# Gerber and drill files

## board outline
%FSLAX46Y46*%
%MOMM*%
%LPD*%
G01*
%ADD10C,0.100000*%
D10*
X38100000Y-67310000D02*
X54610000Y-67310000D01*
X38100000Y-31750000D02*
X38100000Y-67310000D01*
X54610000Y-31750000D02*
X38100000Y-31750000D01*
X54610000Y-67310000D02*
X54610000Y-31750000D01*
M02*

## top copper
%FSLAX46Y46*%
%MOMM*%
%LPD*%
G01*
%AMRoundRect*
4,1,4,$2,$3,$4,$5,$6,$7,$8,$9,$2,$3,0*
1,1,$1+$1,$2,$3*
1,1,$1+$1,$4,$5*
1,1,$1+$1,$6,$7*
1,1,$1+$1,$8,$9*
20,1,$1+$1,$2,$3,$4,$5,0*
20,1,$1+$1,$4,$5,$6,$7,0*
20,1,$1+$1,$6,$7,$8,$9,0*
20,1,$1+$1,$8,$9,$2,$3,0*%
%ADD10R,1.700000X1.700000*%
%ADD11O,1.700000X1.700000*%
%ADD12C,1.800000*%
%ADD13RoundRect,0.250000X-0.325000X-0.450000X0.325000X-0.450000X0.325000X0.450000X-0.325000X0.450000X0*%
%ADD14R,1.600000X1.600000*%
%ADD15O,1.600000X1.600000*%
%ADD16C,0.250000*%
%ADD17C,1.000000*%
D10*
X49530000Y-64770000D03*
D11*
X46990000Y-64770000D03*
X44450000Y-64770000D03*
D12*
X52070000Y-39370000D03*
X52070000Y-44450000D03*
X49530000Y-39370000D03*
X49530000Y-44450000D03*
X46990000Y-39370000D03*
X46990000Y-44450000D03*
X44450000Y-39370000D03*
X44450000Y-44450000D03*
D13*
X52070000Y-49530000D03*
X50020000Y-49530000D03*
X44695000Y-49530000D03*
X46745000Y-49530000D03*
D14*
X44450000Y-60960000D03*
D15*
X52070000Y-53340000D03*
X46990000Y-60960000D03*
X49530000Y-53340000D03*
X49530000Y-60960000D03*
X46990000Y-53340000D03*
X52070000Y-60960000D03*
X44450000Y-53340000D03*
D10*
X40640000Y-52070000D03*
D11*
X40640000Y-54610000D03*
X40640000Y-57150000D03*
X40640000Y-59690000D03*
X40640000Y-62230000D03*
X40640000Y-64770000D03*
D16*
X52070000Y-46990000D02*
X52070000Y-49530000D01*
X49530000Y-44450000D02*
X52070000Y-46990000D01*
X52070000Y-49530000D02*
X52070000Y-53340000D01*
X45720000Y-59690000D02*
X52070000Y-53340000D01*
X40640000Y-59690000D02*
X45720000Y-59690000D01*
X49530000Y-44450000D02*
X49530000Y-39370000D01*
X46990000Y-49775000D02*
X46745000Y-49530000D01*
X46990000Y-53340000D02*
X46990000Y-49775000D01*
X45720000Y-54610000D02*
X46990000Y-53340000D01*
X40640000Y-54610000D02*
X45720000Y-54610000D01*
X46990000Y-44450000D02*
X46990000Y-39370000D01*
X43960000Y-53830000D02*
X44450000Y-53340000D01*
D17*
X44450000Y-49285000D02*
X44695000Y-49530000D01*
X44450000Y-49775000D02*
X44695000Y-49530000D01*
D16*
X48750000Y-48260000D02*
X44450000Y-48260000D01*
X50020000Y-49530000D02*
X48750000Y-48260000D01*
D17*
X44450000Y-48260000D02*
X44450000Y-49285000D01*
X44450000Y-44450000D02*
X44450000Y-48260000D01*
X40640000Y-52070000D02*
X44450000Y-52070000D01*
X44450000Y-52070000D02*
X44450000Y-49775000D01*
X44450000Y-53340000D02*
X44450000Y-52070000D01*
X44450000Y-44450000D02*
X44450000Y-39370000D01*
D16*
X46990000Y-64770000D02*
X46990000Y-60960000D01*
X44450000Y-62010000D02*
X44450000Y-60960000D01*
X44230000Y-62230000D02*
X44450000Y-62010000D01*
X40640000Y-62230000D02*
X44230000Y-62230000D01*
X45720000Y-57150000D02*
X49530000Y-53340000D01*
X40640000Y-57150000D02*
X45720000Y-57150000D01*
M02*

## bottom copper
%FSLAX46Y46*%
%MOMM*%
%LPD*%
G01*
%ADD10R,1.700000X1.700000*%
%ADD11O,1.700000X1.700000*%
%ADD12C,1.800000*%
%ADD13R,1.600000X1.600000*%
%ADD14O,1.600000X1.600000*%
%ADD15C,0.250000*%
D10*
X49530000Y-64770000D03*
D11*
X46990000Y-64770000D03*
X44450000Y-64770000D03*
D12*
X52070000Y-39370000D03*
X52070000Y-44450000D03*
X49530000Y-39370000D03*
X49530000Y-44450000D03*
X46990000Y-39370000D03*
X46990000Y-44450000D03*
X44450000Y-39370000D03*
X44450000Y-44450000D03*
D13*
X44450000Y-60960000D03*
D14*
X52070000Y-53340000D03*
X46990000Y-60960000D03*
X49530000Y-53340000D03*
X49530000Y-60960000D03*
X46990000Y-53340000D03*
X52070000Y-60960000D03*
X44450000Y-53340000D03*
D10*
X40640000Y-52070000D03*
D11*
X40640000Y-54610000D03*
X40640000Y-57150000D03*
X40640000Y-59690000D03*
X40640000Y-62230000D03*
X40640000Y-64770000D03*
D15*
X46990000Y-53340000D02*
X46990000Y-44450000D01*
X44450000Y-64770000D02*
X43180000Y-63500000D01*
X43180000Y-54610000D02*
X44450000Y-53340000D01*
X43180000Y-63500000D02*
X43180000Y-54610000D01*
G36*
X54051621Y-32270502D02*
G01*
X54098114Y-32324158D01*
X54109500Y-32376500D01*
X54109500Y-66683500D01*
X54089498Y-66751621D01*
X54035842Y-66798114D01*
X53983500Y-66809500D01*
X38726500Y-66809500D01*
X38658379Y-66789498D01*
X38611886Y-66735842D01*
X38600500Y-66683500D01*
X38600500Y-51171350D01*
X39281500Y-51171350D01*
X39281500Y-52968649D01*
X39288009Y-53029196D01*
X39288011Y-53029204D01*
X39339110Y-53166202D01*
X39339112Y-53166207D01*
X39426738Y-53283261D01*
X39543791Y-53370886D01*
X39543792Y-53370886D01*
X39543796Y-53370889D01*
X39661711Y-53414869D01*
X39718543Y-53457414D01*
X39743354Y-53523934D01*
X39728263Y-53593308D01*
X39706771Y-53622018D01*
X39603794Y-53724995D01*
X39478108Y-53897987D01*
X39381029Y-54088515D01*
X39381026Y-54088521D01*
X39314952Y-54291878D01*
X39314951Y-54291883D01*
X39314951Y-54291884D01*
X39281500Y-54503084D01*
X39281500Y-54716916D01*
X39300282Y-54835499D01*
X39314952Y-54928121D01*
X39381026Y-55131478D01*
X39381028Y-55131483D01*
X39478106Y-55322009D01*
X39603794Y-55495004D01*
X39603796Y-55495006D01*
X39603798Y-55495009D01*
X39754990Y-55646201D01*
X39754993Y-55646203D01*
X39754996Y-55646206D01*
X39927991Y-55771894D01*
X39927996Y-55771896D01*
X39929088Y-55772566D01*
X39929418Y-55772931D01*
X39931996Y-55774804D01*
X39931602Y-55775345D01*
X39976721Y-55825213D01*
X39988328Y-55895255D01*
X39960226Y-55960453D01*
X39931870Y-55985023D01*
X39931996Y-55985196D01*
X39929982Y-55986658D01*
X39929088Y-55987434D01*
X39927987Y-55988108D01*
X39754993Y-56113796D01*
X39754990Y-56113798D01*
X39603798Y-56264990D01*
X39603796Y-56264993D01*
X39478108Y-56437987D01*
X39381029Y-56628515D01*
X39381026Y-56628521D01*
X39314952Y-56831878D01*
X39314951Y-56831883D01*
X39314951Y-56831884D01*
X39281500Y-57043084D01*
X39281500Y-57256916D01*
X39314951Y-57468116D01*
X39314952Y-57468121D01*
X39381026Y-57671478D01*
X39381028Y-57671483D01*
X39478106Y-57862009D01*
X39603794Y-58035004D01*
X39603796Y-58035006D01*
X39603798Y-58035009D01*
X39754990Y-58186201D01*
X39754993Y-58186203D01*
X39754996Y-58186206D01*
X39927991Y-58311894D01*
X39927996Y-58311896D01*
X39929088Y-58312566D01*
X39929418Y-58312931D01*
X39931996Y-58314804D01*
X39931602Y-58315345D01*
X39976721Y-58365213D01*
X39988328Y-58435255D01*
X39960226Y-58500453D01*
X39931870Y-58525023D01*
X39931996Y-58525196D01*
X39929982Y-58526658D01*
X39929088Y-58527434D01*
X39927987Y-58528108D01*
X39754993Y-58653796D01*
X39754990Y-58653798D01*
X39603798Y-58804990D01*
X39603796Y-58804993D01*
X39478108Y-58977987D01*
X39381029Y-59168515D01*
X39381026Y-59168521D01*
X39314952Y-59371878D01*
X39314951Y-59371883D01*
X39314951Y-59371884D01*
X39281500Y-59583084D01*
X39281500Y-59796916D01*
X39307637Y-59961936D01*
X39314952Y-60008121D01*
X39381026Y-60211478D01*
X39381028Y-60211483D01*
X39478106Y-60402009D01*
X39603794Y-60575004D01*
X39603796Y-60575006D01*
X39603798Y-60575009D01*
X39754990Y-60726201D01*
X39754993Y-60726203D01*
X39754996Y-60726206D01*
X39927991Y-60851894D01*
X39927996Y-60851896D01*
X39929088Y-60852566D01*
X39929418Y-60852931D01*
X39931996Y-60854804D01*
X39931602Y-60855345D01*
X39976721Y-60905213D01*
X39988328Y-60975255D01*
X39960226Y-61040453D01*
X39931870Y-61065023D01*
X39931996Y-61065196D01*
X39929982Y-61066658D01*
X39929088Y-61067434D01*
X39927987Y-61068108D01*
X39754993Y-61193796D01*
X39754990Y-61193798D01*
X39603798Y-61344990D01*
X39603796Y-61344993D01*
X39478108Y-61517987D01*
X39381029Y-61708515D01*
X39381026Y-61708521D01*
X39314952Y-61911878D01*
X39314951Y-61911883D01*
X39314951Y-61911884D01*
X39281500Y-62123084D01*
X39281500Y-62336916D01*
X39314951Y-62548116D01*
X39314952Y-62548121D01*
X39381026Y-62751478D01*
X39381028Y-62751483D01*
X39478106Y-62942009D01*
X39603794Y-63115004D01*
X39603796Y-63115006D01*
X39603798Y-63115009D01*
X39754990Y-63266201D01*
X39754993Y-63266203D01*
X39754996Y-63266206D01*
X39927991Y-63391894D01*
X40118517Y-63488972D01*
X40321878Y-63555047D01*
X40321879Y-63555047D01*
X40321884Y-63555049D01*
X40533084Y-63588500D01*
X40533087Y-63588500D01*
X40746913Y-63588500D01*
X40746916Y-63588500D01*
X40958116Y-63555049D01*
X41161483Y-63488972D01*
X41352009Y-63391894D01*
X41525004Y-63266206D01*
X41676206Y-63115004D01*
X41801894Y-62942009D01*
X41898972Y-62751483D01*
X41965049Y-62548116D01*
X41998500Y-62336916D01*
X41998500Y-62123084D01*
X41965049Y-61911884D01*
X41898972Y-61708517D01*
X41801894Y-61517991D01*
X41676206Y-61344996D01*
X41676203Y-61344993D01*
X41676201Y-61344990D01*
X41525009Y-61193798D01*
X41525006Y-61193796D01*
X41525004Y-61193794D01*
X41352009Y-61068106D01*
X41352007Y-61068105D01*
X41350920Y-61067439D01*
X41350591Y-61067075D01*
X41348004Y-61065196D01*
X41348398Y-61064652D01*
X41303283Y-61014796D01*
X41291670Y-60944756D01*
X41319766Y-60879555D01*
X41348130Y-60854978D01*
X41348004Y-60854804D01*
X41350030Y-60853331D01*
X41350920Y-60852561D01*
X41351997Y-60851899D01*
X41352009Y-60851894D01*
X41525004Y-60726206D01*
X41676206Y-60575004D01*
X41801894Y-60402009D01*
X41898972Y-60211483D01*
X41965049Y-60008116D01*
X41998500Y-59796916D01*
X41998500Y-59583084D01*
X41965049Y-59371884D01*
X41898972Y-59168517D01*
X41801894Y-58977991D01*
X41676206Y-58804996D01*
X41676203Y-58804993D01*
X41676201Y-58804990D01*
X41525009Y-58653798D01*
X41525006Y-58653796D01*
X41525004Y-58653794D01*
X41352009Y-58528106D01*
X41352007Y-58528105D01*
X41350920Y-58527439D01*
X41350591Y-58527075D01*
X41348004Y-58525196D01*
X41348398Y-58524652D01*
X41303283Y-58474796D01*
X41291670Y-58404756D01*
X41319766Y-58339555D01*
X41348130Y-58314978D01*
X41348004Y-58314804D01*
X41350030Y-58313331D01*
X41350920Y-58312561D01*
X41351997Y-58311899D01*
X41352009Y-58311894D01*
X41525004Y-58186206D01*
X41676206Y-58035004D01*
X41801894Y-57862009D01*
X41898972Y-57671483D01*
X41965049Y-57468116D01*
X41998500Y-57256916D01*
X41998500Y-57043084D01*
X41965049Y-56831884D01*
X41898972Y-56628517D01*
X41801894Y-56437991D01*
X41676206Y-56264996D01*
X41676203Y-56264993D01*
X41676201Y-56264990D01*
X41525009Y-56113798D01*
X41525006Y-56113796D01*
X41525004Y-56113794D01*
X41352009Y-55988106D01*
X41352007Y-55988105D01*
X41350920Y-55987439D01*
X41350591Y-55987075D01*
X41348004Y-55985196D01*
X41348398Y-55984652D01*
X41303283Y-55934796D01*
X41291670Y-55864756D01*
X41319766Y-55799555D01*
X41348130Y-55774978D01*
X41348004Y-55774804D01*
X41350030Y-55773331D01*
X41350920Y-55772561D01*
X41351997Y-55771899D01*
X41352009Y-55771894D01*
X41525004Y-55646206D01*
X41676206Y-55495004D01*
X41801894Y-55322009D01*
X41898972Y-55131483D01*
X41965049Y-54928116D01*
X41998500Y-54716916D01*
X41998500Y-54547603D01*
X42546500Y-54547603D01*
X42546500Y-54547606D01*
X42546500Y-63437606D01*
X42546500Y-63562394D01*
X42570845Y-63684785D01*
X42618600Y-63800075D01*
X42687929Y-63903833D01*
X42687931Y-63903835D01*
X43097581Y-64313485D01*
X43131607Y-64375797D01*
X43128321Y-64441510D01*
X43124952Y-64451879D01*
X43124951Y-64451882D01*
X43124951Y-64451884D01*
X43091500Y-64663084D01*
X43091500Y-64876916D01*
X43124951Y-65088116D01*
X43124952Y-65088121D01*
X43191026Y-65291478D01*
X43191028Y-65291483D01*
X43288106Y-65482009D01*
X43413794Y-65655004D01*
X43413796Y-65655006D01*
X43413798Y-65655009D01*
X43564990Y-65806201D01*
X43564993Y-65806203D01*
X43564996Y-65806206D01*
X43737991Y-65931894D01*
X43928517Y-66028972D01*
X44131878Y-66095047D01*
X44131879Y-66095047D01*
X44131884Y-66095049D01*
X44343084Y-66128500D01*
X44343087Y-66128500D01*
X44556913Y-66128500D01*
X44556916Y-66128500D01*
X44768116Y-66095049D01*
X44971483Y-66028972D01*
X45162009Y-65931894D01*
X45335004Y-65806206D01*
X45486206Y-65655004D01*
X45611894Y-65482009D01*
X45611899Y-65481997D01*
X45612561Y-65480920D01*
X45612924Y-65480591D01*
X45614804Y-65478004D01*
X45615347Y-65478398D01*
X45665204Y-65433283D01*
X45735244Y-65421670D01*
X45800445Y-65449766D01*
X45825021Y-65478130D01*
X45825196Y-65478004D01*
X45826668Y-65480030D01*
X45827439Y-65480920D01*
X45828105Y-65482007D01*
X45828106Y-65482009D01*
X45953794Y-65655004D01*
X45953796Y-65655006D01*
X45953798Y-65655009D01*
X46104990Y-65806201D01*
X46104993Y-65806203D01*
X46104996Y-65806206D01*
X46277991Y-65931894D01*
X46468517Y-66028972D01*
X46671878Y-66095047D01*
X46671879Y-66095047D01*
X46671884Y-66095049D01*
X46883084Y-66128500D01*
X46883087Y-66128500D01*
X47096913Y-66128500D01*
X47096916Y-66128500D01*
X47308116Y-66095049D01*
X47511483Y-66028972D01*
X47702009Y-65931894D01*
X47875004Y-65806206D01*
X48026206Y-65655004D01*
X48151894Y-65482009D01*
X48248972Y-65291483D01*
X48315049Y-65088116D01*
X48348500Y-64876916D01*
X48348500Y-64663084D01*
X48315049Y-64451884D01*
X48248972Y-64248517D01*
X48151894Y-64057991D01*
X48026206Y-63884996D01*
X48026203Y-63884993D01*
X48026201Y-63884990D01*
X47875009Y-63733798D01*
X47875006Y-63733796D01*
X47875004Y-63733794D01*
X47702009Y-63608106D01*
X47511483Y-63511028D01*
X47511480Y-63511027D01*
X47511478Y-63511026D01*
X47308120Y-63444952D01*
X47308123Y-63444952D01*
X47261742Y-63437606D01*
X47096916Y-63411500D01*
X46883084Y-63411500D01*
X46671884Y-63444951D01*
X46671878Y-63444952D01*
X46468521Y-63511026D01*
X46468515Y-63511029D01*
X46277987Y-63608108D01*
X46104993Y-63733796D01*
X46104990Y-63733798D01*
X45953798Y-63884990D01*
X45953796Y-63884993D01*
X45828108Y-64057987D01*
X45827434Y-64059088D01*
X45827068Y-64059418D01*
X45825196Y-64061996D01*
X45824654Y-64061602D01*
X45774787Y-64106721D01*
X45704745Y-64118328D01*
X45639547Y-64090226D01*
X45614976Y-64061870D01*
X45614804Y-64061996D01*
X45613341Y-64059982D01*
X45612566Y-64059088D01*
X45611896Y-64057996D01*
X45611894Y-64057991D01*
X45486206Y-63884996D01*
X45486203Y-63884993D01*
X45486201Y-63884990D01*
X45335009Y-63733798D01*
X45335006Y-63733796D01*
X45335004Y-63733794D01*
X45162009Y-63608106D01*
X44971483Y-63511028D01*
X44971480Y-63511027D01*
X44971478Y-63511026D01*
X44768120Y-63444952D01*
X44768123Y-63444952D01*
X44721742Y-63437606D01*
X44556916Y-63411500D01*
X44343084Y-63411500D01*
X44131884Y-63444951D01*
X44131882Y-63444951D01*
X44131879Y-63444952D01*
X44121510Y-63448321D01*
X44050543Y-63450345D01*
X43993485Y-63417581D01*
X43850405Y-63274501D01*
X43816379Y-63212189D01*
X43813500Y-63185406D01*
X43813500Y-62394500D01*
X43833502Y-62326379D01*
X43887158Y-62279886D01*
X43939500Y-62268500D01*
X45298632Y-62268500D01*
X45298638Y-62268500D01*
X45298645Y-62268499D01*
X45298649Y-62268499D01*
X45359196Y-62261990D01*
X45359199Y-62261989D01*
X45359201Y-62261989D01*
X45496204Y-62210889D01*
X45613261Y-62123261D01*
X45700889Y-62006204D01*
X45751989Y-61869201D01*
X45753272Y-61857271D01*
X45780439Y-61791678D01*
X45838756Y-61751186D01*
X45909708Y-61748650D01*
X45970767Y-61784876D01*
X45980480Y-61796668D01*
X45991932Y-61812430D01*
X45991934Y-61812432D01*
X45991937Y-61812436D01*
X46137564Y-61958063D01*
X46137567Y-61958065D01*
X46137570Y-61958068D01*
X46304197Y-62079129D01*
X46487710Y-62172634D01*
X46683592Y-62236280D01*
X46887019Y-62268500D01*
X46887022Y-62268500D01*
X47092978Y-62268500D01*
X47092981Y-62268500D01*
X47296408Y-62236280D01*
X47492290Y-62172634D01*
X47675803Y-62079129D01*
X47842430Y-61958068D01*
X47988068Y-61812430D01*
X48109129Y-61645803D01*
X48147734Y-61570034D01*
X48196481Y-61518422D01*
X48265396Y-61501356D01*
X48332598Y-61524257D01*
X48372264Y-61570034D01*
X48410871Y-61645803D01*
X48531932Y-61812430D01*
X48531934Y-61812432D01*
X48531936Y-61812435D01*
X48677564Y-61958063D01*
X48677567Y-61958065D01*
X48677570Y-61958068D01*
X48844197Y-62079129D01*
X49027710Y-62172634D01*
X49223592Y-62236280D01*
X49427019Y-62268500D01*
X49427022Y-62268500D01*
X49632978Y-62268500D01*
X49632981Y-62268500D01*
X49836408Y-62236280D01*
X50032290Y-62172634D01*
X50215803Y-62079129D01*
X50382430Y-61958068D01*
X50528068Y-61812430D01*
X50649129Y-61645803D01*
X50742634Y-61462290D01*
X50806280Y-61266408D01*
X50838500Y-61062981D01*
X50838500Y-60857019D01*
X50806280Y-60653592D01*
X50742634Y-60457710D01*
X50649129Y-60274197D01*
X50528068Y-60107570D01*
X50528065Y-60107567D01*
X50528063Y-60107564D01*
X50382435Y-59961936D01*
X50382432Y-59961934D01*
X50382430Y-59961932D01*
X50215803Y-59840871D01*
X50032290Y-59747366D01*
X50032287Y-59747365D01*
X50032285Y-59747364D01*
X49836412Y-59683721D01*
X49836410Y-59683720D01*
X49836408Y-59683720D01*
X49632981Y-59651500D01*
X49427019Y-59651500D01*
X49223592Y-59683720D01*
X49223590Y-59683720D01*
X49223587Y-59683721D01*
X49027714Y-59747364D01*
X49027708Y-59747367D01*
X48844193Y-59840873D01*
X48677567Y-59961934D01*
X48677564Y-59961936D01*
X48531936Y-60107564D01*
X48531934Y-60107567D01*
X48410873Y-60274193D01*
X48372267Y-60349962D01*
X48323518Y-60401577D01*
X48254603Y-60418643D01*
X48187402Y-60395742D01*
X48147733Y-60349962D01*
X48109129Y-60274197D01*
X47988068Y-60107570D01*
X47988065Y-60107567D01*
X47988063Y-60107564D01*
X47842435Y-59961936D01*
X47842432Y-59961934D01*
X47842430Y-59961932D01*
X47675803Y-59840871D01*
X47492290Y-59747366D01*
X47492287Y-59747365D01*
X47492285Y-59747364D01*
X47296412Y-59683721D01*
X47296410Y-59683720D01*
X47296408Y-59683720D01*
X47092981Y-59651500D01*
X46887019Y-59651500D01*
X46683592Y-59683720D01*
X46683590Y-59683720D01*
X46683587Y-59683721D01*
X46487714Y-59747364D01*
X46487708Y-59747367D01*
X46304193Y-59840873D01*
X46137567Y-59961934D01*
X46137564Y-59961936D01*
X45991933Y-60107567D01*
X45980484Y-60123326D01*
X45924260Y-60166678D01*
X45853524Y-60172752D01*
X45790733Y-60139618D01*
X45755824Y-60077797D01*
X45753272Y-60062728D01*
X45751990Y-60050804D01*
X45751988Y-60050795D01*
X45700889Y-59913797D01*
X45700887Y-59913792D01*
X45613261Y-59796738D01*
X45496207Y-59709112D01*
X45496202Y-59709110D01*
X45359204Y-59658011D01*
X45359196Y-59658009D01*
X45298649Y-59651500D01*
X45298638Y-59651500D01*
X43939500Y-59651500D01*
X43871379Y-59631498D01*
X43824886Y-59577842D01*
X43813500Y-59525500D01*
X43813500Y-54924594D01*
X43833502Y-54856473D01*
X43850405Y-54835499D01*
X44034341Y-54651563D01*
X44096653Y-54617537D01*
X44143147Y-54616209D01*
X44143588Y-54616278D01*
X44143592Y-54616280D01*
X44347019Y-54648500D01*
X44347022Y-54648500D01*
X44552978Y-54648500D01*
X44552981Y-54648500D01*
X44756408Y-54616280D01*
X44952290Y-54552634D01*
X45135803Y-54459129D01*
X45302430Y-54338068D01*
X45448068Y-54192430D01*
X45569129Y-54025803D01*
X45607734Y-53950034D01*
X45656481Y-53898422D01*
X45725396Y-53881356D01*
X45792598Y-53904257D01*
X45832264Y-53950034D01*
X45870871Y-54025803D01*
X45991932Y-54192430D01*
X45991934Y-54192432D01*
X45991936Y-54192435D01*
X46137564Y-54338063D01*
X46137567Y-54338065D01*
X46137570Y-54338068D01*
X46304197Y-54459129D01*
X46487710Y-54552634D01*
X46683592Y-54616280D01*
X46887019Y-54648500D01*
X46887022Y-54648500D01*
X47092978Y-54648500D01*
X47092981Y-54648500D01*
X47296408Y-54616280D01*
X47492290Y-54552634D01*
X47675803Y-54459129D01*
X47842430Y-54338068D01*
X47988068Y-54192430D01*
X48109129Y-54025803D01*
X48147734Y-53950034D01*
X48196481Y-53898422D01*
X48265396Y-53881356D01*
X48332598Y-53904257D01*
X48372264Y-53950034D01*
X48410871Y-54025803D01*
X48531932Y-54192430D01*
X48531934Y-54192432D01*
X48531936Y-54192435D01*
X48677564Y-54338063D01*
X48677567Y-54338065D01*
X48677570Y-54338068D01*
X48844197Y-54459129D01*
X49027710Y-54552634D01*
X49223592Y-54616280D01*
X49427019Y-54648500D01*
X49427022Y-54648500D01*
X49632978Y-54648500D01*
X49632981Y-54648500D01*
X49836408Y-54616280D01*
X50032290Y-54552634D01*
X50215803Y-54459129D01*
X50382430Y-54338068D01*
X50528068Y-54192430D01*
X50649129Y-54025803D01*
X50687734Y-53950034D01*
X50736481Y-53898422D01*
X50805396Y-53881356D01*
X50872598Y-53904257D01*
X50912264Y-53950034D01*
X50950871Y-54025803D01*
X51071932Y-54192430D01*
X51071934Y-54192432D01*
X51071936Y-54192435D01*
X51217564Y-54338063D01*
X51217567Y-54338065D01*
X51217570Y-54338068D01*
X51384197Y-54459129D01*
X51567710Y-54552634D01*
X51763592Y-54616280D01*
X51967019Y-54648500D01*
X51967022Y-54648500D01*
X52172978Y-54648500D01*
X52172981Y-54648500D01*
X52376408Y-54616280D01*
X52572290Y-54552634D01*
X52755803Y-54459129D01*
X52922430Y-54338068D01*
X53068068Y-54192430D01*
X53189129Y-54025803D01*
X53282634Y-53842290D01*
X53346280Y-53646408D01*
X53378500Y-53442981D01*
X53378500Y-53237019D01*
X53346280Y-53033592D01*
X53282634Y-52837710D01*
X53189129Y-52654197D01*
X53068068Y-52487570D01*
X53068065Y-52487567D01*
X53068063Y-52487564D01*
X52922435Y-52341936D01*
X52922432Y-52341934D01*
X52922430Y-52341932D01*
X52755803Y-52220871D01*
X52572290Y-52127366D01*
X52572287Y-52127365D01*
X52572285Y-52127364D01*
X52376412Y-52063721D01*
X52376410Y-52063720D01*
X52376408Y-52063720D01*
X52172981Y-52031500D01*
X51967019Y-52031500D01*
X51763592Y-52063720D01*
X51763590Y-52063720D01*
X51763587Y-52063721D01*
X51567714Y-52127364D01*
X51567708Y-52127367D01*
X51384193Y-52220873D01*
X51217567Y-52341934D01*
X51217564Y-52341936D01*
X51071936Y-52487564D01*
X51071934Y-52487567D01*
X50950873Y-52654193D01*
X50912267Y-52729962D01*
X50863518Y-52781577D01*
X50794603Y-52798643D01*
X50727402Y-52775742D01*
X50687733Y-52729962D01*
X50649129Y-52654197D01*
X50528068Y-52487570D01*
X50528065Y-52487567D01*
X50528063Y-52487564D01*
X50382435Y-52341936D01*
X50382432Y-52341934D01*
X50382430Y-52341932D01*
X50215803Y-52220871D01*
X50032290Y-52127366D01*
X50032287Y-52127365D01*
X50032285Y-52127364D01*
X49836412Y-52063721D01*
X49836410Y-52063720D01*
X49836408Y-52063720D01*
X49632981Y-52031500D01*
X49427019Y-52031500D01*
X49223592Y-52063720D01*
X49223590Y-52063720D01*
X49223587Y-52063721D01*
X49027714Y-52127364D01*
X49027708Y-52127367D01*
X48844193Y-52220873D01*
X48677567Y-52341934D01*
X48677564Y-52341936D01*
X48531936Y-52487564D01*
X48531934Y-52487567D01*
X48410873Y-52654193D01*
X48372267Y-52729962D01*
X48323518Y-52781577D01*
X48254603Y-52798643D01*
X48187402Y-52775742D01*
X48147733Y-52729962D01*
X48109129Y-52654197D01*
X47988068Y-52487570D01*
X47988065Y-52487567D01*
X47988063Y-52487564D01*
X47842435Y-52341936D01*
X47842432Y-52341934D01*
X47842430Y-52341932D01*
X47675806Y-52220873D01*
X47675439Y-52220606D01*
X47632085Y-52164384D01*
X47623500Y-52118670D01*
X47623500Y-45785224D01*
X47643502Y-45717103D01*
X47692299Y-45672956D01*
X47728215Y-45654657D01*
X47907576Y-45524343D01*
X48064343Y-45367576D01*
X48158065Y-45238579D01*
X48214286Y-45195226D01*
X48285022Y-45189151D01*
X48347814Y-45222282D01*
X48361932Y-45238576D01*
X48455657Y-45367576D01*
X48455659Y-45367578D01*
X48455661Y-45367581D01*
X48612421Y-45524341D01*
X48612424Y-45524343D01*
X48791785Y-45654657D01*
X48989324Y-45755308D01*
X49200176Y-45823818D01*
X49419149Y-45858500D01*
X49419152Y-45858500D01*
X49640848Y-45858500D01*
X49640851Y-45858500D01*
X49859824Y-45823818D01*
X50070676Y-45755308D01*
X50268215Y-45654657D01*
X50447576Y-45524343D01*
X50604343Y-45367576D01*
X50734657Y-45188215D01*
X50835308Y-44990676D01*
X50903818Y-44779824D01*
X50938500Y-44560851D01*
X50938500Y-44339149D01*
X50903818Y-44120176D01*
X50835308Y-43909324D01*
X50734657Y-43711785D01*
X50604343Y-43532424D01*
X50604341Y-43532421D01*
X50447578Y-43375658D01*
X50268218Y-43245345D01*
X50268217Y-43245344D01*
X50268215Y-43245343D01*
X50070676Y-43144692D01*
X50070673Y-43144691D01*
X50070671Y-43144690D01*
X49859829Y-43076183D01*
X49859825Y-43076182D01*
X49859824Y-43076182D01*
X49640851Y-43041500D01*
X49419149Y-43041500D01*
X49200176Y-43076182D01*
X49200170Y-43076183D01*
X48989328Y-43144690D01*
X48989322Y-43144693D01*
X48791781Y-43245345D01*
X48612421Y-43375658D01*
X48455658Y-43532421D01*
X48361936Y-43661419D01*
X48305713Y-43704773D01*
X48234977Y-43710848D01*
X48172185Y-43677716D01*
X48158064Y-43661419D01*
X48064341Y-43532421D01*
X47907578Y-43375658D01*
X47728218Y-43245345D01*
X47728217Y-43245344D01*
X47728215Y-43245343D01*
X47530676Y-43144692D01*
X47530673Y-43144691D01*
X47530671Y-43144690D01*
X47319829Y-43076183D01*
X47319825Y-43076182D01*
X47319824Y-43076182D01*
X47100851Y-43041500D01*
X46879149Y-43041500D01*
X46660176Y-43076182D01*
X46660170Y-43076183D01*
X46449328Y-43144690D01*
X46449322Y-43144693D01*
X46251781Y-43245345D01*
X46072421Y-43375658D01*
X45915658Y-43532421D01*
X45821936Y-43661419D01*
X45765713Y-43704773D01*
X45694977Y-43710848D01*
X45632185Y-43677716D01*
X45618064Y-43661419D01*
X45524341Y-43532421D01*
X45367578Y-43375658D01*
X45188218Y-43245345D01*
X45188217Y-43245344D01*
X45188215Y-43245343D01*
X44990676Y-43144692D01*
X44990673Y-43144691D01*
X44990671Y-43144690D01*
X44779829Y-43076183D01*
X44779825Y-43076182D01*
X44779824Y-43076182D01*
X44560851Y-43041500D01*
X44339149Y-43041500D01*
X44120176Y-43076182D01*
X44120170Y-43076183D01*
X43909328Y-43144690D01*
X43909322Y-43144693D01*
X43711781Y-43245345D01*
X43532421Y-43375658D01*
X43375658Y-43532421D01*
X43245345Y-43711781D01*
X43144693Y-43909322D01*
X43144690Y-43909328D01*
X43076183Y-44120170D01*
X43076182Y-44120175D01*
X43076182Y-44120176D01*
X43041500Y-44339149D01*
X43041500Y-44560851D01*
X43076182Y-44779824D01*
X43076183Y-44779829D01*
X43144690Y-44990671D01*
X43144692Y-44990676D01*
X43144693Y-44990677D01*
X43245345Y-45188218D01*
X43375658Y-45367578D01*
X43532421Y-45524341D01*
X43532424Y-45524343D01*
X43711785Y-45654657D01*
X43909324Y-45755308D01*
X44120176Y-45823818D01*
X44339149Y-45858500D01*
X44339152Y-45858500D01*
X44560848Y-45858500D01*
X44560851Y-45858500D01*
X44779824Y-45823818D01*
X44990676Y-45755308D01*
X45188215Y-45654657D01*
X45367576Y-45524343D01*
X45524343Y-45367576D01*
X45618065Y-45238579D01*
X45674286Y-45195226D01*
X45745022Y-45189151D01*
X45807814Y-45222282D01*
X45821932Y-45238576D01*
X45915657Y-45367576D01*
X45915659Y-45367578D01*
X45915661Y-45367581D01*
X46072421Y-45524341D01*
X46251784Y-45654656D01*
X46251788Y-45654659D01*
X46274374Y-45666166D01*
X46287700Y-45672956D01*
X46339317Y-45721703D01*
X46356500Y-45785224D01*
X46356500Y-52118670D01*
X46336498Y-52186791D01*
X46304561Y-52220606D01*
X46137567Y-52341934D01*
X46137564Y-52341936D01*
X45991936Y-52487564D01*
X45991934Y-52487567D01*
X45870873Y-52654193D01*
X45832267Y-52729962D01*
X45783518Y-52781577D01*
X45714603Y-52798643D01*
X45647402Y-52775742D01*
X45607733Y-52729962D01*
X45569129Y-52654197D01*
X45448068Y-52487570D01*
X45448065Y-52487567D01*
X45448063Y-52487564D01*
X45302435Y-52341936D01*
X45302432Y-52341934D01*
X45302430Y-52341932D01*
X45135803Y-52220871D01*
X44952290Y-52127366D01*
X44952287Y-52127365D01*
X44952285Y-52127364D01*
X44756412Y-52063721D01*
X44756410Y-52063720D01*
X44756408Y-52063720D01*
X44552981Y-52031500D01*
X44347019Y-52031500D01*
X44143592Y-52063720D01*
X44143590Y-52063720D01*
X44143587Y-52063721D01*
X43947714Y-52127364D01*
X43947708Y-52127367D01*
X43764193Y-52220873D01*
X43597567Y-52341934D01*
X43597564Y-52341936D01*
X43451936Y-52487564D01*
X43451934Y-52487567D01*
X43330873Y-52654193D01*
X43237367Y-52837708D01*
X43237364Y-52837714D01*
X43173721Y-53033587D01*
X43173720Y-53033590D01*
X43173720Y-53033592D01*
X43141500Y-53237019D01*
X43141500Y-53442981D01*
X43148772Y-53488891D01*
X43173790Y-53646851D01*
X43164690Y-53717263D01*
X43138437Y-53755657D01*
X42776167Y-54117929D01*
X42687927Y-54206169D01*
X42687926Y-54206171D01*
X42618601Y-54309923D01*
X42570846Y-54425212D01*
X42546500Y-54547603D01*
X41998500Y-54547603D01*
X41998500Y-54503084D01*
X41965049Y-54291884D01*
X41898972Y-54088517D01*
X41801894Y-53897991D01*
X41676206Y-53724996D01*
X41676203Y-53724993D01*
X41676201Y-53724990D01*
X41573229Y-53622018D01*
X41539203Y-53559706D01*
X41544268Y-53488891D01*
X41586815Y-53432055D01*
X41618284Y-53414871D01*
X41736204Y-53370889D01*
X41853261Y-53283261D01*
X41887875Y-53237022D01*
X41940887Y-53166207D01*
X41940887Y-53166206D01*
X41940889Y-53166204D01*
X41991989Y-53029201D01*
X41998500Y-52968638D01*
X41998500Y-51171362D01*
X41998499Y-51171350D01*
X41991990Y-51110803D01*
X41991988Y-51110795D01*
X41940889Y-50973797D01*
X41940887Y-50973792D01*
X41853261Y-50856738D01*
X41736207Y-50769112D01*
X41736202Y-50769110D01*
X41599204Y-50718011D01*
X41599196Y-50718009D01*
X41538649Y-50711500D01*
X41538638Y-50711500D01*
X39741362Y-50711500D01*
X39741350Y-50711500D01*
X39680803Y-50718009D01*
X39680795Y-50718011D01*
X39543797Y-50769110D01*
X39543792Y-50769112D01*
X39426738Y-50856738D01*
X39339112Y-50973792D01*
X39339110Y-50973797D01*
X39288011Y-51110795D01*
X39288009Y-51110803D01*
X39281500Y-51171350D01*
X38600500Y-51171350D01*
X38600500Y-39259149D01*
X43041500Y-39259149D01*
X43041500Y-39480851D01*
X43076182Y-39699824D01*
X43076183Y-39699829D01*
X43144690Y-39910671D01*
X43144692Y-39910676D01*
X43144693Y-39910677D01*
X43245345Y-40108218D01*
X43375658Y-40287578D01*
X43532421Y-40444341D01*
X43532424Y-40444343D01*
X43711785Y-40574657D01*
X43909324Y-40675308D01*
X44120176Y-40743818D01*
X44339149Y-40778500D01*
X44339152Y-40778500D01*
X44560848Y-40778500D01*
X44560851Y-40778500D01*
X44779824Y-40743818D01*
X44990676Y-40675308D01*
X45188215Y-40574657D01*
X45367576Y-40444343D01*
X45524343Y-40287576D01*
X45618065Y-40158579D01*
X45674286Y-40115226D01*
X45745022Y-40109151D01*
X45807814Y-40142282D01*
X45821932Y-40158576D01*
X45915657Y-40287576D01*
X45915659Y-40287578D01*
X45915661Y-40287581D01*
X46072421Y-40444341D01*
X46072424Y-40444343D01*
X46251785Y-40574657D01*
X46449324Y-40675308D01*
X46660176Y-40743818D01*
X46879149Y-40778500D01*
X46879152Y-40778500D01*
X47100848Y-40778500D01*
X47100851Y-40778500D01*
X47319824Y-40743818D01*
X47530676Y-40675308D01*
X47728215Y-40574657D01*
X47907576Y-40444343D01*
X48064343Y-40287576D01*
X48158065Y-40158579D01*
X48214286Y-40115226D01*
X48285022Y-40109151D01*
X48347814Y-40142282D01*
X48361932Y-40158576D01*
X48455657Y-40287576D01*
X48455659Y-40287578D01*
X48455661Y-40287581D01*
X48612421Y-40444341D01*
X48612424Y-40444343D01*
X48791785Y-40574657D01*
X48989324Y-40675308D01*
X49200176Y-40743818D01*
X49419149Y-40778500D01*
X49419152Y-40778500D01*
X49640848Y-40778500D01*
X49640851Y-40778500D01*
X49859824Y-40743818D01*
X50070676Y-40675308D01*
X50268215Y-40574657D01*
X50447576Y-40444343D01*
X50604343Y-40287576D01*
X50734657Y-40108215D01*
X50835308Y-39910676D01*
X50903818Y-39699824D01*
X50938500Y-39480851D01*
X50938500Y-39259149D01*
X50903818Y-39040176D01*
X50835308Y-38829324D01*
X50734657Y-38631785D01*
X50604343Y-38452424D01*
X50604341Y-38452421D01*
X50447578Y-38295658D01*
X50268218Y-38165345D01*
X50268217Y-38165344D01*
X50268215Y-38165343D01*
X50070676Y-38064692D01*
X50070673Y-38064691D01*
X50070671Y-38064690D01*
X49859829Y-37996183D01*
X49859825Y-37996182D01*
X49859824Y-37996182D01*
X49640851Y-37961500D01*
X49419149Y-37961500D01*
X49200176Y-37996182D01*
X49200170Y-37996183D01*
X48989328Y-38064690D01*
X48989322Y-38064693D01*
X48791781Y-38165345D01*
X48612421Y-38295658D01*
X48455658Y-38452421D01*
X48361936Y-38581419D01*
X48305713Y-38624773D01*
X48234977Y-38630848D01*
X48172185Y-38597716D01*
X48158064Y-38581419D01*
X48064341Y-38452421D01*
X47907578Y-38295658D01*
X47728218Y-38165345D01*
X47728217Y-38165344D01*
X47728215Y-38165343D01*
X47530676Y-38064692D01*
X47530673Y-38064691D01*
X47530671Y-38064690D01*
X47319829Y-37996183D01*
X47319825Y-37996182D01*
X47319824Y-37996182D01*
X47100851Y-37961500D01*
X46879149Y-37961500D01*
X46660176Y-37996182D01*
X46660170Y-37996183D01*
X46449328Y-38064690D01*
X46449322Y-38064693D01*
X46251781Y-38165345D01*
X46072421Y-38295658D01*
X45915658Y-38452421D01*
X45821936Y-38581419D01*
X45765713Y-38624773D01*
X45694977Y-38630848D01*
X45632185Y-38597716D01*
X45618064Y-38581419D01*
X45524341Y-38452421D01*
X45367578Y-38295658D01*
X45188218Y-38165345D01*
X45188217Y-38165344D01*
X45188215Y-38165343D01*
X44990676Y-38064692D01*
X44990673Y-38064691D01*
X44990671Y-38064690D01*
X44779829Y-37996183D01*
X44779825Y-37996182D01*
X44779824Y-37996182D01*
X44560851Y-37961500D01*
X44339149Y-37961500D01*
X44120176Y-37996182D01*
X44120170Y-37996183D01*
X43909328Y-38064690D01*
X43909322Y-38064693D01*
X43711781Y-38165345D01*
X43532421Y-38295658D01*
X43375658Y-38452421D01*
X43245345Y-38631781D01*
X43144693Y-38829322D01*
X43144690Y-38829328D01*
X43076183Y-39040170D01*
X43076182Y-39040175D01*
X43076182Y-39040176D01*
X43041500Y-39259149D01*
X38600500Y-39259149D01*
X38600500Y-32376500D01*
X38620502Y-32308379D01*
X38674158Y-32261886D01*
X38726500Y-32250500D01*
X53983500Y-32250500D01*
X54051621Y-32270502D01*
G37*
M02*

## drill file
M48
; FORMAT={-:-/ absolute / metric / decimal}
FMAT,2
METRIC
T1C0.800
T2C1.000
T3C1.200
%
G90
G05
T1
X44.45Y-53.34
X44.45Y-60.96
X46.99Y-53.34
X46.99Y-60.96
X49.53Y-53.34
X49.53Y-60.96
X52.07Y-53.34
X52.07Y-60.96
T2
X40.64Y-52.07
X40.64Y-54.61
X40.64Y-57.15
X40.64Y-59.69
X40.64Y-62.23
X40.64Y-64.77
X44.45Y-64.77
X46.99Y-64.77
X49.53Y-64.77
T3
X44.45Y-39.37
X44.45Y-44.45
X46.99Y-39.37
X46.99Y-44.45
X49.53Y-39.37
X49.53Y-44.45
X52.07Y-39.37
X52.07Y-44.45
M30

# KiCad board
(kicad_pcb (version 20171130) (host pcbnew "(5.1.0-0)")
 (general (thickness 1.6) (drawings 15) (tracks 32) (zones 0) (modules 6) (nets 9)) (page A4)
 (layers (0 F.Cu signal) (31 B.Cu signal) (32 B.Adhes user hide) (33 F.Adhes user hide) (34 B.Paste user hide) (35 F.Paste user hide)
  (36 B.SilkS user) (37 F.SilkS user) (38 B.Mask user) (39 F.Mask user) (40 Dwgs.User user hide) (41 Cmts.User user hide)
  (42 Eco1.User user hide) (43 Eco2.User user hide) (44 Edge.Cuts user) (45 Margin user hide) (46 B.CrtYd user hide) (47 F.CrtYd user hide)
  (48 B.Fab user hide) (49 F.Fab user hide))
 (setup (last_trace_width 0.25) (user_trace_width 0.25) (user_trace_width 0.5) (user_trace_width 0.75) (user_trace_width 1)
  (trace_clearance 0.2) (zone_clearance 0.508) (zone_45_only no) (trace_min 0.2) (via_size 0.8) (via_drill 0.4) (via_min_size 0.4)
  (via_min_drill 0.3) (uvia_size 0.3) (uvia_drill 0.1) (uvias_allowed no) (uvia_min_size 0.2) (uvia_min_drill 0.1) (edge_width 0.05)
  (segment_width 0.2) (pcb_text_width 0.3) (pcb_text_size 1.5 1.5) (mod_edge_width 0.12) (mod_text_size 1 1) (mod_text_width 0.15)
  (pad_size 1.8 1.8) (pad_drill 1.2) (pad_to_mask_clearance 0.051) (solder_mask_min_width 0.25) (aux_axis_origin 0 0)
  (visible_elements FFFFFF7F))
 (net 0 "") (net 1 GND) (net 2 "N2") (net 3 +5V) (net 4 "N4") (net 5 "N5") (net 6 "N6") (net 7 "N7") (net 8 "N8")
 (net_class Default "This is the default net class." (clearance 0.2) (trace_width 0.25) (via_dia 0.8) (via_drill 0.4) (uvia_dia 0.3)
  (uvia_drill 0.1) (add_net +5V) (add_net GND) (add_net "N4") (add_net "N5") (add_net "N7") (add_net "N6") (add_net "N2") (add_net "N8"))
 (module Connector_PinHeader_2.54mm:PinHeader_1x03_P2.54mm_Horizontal (layer F.Cu) (at 49.53 64.77 270)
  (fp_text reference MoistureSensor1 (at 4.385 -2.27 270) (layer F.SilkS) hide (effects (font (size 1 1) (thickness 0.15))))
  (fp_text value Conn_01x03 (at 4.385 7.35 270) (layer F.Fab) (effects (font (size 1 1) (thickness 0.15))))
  (pad 1 thru_hole rect (at 0 0 270) (size 1.7 1.7) (drill 1) (layers *.Cu *.Mask) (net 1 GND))
  (pad 2 thru_hole oval (at 0 2.54 270) (size 1.7 1.7) (drill 1) (layers *.Cu *.Mask) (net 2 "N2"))
  (pad 3 thru_hole oval (at 0 5.08 270) (size 1.7 1.7) (drill 1) (layers *.Cu *.Mask) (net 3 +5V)))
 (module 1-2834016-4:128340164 (layer F.Cu) (at 52.07 39.37 180)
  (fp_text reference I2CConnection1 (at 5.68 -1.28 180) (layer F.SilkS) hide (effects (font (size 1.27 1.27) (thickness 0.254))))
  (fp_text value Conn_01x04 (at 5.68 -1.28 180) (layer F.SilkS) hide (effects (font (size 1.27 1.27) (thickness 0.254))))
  (pad "" thru_hole circle (at 0 0 180) (size 1.8 1.8) (drill 1.2) (layers *.Cu *.Mask) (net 1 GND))
  (pad 1 thru_hole circle (at 0 -5.08 180) (size 1.8 1.8) (drill 1.2) (layers *.Cu *.Mask) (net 1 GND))
  (pad "" thru_hole circle (at 2.54 0 180) (size 1.8 1.8) (drill 1.2) (layers *.Cu *.Mask) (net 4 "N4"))
  (pad 2 thru_hole circle (at 2.54 -5.08 180) (size 1.8 1.8) (drill 1.2) (layers *.Cu *.Mask) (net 4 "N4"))
  (pad "" thru_hole circle (at 5.08 0 180) (size 1.8 1.8) (drill 1.2) (layers *.Cu *.Mask) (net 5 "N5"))
  (pad 3 thru_hole circle (at 5.08 -5.08 180) (size 1.8 1.8) (drill 1.2) (layers *.Cu *.Mask) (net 5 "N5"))
  (pad "" thru_hole circle (at 7.62 0 180) (size 1.8 1.8) (drill 1.2) (layers *.Cu *.Mask) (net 3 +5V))
  (pad 4 thru_hole circle (at 7.62 -5.08 180) (size 1.8 1.8) (drill 1.2) (layers *.Cu *.Mask) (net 3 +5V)))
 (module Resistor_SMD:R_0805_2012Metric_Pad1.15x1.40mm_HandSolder (layer F.Cu) (at 51.045 49.53)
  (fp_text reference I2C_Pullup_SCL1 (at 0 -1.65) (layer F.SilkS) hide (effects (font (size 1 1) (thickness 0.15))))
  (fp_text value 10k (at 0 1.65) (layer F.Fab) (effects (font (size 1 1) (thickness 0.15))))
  (pad 2 smd roundrect (at 1.025 0) (size 1.15 1.4) (layers F.Cu F.Paste F.Mask) (roundrect_rratio 0.217391) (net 4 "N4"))
  (pad 1 smd roundrect (at -1.025 0) (size 1.15 1.4) (layers F.Cu F.Paste F.Mask) (roundrect_rratio 0.217391) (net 3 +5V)))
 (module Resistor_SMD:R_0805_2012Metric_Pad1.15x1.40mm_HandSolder (layer F.Cu) (at 45.72 49.53)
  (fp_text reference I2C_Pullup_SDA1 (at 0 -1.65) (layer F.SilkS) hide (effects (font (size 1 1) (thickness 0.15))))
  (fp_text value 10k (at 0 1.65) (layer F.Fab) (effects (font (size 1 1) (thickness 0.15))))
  (pad 1 smd roundrect (at -1.025 0) (size 1.15 1.4) (layers F.Cu F.Paste F.Mask) (roundrect_rratio 0.217391) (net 3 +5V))
  (pad 2 smd roundrect (at 1.025 0) (size 1.15 1.4) (layers F.Cu F.Paste F.Mask) (roundrect_rratio 0.217391) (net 5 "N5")))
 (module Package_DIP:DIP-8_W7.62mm (layer F.Cu) (at 44.45 60.96 90)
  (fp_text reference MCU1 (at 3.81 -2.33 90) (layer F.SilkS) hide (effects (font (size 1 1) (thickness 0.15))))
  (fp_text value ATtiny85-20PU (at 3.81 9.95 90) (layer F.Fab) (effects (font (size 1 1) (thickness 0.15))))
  (pad 1 thru_hole rect (at 0 0 90) (size 1.6 1.6) (drill 0.8) (layers *.Cu *.Mask) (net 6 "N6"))
  (pad 5 thru_hole oval (at 7.62 7.62 90) (size 1.6 1.6) (drill 0.8) (layers *.Cu *.Mask) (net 4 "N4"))
  (pad 2 thru_hole oval (at 0 2.54 90) (size 1.6 1.6) (drill 0.8) (layers *.Cu *.Mask) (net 2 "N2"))
  (pad 6 thru_hole oval (at 7.62 5.08 90) (size 1.6 1.6) (drill 0.8) (layers *.Cu *.Mask) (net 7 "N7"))
  (pad 3 thru_hole oval (at 0 5.08 90) (size 1.6 1.6) (drill 0.8) (layers *.Cu *.Mask) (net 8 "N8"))
  (pad 7 thru_hole oval (at 7.62 2.54 90) (size 1.6 1.6) (drill 0.8) (layers *.Cu *.Mask) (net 5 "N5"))
  (pad 4 thru_hole oval (at 0 7.62 90) (size 1.6 1.6) (drill 0.8) (layers *.Cu *.Mask) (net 1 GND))
  (pad 8 thru_hole oval (at 7.62 0 90) (size 1.6 1.6) (drill 0.8) (layers *.Cu *.Mask) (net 3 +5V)))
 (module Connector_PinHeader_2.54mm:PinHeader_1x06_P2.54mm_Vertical (layer F.Cu) (at 40.64 52.07)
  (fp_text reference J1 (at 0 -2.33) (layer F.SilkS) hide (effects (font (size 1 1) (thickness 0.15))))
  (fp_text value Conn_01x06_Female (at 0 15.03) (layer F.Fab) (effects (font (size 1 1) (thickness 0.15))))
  (pad 1 thru_hole rect (at 0 0) (size 1.7 1.7) (drill 1) (layers *.Cu *.Mask) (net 3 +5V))
  (pad 2 thru_hole oval (at 0 2.54) (size 1.7 1.7) (drill 1) (layers *.Cu *.Mask) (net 5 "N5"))
  (pad 3 thru_hole oval (at 0 5.08) (size 1.7 1.7) (drill 1) (layers *.Cu *.Mask) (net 7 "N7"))
  (pad 4 thru_hole oval (at 0 7.62) (size 1.7 1.7) (drill 1) (layers *.Cu *.Mask) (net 4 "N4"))
  (pad 5 thru_hole oval (at 0 10.16) (size 1.7 1.7) (drill 1) (layers *.Cu *.Mask) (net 6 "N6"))
  (pad 6 thru_hole oval (at 0 12.7) (size 1.7 1.7) (drill 1) (layers *.Cu *.Mask) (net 1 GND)))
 (gr_line (start 38.1 67.31) (end 54.61 67.31) (layer Edge.Cuts) (width 0.1))
 (gr_line (start 38.1 31.75) (end 38.1 67.31) (layer Edge.Cuts) (width 0.1))
 (gr_line (start 54.61 31.75) (end 38.1 31.75) (layer Edge.Cuts) (width 0.1))
 (gr_line (start 54.61 67.31) (end 54.61 31.75) (layer Edge.Cuts) (width 0.1))
 (segment (start 52.07 46.99) (end 52.07 49.53) (width 0.25) (layer F.Cu) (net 4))
 (segment (start 49.53 44.45) (end 52.07 46.99) (width 0.25) (layer F.Cu) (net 4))
 (segment (start 52.07 49.53) (end 52.07 53.34) (width 0.25) (layer F.Cu) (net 4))
 (segment (start 45.72 59.69) (end 52.07 53.34) (width 0.25) (layer F.Cu) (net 4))
 (segment (start 40.64 59.69) (end 45.72 59.69) (width 0.25) (layer F.Cu) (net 4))
 (segment (start 49.53 44.45) (end 49.53 39.37) (width 0.25) (layer F.Cu) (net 4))
 (segment (start 46.99 49.775) (end 46.745 49.53) (width 0.25) (layer F.Cu) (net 5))
 (segment (start 46.99 53.34) (end 46.99 49.775) (width 0.25) (layer F.Cu) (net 5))
 (segment (start 46.99 53.34) (end 46.99 44.45) (width 0.25) (layer B.Cu) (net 5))
 (segment (start 45.72 54.61) (end 46.99 53.34) (width 0.25) (layer F.Cu) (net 5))
 (segment (start 40.64 54.61) (end 45.72 54.61) (width 0.25) (layer F.Cu) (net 5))
 (segment (start 46.99 44.45) (end 46.99 39.37) (width 0.25) (layer F.Cu) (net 5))
 (segment (start 43.96 53.83) (end 44.45 53.34) (width 0.25) (layer F.Cu) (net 3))
 (segment (start 44.45 49.285) (end 44.695 49.53) (width 1) (layer F.Cu) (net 3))
 (segment (start 44.45 49.775) (end 44.695 49.53) (width 1) (layer F.Cu) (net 3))
 (segment (start 48.75 48.26) (end 44.45 48.26) (width 0.25) (layer F.Cu) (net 3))
 (segment (start 50.02 49.53) (end 48.75 48.26) (width 0.25) (layer F.Cu) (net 3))
 (segment (start 44.45 48.26) (end 44.45 49.285) (width 1) (layer F.Cu) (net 3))
 (segment (start 44.45 44.45) (end 44.45 48.26) (width 1) (layer F.Cu) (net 3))
 (segment (start 40.64 52.07) (end 44.45 52.07) (width 1) (layer F.Cu) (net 3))
 (segment (start 44.45 52.07) (end 44.45 49.775) (width 1) (layer F.Cu) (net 3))
 (segment (start 44.45 53.34) (end 44.45 52.07) (width 1) (layer F.Cu) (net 3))
 (segment (start 44.45 64.77) (end 43.18 63.5) (width 0.25) (layer B.Cu) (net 3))
 (segment (start 43.18 54.61) (end 44.45 53.34) (width 0.25) (layer B.Cu) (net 3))
 (segment (start 43.18 63.5) (end 43.18 54.61) (width 0.25) (layer B.Cu) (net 3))
 (segment (start 44.45 44.45) (end 44.45 39.37) (width 1) (layer F.Cu) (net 3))
 (segment (start 46.99 64.77) (end 46.99 60.96) (width 0.25) (layer F.Cu) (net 2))
 (segment (start 44.45 62.01) (end 44.45 60.96) (width 0.25) (layer F.Cu) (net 6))
 (segment (start 44.23 62.23) (end 44.45 62.01) (width 0.25) (layer F.Cu) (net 6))
 (segment (start 40.64 62.23) (end 44.23 62.23) (width 0.25) (layer F.Cu) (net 6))
 (segment (start 45.72 57.15) (end 49.53 53.34) (width 0.25) (layer F.Cu) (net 7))
 (segment (start 40.64 57.15) (end 45.72 57.15) (width 0.25) (layer F.Cu) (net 7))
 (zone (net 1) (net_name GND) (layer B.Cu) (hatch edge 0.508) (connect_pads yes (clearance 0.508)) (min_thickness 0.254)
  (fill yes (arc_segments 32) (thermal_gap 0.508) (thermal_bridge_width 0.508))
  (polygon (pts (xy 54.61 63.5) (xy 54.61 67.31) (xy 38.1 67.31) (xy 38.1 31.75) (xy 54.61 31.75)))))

